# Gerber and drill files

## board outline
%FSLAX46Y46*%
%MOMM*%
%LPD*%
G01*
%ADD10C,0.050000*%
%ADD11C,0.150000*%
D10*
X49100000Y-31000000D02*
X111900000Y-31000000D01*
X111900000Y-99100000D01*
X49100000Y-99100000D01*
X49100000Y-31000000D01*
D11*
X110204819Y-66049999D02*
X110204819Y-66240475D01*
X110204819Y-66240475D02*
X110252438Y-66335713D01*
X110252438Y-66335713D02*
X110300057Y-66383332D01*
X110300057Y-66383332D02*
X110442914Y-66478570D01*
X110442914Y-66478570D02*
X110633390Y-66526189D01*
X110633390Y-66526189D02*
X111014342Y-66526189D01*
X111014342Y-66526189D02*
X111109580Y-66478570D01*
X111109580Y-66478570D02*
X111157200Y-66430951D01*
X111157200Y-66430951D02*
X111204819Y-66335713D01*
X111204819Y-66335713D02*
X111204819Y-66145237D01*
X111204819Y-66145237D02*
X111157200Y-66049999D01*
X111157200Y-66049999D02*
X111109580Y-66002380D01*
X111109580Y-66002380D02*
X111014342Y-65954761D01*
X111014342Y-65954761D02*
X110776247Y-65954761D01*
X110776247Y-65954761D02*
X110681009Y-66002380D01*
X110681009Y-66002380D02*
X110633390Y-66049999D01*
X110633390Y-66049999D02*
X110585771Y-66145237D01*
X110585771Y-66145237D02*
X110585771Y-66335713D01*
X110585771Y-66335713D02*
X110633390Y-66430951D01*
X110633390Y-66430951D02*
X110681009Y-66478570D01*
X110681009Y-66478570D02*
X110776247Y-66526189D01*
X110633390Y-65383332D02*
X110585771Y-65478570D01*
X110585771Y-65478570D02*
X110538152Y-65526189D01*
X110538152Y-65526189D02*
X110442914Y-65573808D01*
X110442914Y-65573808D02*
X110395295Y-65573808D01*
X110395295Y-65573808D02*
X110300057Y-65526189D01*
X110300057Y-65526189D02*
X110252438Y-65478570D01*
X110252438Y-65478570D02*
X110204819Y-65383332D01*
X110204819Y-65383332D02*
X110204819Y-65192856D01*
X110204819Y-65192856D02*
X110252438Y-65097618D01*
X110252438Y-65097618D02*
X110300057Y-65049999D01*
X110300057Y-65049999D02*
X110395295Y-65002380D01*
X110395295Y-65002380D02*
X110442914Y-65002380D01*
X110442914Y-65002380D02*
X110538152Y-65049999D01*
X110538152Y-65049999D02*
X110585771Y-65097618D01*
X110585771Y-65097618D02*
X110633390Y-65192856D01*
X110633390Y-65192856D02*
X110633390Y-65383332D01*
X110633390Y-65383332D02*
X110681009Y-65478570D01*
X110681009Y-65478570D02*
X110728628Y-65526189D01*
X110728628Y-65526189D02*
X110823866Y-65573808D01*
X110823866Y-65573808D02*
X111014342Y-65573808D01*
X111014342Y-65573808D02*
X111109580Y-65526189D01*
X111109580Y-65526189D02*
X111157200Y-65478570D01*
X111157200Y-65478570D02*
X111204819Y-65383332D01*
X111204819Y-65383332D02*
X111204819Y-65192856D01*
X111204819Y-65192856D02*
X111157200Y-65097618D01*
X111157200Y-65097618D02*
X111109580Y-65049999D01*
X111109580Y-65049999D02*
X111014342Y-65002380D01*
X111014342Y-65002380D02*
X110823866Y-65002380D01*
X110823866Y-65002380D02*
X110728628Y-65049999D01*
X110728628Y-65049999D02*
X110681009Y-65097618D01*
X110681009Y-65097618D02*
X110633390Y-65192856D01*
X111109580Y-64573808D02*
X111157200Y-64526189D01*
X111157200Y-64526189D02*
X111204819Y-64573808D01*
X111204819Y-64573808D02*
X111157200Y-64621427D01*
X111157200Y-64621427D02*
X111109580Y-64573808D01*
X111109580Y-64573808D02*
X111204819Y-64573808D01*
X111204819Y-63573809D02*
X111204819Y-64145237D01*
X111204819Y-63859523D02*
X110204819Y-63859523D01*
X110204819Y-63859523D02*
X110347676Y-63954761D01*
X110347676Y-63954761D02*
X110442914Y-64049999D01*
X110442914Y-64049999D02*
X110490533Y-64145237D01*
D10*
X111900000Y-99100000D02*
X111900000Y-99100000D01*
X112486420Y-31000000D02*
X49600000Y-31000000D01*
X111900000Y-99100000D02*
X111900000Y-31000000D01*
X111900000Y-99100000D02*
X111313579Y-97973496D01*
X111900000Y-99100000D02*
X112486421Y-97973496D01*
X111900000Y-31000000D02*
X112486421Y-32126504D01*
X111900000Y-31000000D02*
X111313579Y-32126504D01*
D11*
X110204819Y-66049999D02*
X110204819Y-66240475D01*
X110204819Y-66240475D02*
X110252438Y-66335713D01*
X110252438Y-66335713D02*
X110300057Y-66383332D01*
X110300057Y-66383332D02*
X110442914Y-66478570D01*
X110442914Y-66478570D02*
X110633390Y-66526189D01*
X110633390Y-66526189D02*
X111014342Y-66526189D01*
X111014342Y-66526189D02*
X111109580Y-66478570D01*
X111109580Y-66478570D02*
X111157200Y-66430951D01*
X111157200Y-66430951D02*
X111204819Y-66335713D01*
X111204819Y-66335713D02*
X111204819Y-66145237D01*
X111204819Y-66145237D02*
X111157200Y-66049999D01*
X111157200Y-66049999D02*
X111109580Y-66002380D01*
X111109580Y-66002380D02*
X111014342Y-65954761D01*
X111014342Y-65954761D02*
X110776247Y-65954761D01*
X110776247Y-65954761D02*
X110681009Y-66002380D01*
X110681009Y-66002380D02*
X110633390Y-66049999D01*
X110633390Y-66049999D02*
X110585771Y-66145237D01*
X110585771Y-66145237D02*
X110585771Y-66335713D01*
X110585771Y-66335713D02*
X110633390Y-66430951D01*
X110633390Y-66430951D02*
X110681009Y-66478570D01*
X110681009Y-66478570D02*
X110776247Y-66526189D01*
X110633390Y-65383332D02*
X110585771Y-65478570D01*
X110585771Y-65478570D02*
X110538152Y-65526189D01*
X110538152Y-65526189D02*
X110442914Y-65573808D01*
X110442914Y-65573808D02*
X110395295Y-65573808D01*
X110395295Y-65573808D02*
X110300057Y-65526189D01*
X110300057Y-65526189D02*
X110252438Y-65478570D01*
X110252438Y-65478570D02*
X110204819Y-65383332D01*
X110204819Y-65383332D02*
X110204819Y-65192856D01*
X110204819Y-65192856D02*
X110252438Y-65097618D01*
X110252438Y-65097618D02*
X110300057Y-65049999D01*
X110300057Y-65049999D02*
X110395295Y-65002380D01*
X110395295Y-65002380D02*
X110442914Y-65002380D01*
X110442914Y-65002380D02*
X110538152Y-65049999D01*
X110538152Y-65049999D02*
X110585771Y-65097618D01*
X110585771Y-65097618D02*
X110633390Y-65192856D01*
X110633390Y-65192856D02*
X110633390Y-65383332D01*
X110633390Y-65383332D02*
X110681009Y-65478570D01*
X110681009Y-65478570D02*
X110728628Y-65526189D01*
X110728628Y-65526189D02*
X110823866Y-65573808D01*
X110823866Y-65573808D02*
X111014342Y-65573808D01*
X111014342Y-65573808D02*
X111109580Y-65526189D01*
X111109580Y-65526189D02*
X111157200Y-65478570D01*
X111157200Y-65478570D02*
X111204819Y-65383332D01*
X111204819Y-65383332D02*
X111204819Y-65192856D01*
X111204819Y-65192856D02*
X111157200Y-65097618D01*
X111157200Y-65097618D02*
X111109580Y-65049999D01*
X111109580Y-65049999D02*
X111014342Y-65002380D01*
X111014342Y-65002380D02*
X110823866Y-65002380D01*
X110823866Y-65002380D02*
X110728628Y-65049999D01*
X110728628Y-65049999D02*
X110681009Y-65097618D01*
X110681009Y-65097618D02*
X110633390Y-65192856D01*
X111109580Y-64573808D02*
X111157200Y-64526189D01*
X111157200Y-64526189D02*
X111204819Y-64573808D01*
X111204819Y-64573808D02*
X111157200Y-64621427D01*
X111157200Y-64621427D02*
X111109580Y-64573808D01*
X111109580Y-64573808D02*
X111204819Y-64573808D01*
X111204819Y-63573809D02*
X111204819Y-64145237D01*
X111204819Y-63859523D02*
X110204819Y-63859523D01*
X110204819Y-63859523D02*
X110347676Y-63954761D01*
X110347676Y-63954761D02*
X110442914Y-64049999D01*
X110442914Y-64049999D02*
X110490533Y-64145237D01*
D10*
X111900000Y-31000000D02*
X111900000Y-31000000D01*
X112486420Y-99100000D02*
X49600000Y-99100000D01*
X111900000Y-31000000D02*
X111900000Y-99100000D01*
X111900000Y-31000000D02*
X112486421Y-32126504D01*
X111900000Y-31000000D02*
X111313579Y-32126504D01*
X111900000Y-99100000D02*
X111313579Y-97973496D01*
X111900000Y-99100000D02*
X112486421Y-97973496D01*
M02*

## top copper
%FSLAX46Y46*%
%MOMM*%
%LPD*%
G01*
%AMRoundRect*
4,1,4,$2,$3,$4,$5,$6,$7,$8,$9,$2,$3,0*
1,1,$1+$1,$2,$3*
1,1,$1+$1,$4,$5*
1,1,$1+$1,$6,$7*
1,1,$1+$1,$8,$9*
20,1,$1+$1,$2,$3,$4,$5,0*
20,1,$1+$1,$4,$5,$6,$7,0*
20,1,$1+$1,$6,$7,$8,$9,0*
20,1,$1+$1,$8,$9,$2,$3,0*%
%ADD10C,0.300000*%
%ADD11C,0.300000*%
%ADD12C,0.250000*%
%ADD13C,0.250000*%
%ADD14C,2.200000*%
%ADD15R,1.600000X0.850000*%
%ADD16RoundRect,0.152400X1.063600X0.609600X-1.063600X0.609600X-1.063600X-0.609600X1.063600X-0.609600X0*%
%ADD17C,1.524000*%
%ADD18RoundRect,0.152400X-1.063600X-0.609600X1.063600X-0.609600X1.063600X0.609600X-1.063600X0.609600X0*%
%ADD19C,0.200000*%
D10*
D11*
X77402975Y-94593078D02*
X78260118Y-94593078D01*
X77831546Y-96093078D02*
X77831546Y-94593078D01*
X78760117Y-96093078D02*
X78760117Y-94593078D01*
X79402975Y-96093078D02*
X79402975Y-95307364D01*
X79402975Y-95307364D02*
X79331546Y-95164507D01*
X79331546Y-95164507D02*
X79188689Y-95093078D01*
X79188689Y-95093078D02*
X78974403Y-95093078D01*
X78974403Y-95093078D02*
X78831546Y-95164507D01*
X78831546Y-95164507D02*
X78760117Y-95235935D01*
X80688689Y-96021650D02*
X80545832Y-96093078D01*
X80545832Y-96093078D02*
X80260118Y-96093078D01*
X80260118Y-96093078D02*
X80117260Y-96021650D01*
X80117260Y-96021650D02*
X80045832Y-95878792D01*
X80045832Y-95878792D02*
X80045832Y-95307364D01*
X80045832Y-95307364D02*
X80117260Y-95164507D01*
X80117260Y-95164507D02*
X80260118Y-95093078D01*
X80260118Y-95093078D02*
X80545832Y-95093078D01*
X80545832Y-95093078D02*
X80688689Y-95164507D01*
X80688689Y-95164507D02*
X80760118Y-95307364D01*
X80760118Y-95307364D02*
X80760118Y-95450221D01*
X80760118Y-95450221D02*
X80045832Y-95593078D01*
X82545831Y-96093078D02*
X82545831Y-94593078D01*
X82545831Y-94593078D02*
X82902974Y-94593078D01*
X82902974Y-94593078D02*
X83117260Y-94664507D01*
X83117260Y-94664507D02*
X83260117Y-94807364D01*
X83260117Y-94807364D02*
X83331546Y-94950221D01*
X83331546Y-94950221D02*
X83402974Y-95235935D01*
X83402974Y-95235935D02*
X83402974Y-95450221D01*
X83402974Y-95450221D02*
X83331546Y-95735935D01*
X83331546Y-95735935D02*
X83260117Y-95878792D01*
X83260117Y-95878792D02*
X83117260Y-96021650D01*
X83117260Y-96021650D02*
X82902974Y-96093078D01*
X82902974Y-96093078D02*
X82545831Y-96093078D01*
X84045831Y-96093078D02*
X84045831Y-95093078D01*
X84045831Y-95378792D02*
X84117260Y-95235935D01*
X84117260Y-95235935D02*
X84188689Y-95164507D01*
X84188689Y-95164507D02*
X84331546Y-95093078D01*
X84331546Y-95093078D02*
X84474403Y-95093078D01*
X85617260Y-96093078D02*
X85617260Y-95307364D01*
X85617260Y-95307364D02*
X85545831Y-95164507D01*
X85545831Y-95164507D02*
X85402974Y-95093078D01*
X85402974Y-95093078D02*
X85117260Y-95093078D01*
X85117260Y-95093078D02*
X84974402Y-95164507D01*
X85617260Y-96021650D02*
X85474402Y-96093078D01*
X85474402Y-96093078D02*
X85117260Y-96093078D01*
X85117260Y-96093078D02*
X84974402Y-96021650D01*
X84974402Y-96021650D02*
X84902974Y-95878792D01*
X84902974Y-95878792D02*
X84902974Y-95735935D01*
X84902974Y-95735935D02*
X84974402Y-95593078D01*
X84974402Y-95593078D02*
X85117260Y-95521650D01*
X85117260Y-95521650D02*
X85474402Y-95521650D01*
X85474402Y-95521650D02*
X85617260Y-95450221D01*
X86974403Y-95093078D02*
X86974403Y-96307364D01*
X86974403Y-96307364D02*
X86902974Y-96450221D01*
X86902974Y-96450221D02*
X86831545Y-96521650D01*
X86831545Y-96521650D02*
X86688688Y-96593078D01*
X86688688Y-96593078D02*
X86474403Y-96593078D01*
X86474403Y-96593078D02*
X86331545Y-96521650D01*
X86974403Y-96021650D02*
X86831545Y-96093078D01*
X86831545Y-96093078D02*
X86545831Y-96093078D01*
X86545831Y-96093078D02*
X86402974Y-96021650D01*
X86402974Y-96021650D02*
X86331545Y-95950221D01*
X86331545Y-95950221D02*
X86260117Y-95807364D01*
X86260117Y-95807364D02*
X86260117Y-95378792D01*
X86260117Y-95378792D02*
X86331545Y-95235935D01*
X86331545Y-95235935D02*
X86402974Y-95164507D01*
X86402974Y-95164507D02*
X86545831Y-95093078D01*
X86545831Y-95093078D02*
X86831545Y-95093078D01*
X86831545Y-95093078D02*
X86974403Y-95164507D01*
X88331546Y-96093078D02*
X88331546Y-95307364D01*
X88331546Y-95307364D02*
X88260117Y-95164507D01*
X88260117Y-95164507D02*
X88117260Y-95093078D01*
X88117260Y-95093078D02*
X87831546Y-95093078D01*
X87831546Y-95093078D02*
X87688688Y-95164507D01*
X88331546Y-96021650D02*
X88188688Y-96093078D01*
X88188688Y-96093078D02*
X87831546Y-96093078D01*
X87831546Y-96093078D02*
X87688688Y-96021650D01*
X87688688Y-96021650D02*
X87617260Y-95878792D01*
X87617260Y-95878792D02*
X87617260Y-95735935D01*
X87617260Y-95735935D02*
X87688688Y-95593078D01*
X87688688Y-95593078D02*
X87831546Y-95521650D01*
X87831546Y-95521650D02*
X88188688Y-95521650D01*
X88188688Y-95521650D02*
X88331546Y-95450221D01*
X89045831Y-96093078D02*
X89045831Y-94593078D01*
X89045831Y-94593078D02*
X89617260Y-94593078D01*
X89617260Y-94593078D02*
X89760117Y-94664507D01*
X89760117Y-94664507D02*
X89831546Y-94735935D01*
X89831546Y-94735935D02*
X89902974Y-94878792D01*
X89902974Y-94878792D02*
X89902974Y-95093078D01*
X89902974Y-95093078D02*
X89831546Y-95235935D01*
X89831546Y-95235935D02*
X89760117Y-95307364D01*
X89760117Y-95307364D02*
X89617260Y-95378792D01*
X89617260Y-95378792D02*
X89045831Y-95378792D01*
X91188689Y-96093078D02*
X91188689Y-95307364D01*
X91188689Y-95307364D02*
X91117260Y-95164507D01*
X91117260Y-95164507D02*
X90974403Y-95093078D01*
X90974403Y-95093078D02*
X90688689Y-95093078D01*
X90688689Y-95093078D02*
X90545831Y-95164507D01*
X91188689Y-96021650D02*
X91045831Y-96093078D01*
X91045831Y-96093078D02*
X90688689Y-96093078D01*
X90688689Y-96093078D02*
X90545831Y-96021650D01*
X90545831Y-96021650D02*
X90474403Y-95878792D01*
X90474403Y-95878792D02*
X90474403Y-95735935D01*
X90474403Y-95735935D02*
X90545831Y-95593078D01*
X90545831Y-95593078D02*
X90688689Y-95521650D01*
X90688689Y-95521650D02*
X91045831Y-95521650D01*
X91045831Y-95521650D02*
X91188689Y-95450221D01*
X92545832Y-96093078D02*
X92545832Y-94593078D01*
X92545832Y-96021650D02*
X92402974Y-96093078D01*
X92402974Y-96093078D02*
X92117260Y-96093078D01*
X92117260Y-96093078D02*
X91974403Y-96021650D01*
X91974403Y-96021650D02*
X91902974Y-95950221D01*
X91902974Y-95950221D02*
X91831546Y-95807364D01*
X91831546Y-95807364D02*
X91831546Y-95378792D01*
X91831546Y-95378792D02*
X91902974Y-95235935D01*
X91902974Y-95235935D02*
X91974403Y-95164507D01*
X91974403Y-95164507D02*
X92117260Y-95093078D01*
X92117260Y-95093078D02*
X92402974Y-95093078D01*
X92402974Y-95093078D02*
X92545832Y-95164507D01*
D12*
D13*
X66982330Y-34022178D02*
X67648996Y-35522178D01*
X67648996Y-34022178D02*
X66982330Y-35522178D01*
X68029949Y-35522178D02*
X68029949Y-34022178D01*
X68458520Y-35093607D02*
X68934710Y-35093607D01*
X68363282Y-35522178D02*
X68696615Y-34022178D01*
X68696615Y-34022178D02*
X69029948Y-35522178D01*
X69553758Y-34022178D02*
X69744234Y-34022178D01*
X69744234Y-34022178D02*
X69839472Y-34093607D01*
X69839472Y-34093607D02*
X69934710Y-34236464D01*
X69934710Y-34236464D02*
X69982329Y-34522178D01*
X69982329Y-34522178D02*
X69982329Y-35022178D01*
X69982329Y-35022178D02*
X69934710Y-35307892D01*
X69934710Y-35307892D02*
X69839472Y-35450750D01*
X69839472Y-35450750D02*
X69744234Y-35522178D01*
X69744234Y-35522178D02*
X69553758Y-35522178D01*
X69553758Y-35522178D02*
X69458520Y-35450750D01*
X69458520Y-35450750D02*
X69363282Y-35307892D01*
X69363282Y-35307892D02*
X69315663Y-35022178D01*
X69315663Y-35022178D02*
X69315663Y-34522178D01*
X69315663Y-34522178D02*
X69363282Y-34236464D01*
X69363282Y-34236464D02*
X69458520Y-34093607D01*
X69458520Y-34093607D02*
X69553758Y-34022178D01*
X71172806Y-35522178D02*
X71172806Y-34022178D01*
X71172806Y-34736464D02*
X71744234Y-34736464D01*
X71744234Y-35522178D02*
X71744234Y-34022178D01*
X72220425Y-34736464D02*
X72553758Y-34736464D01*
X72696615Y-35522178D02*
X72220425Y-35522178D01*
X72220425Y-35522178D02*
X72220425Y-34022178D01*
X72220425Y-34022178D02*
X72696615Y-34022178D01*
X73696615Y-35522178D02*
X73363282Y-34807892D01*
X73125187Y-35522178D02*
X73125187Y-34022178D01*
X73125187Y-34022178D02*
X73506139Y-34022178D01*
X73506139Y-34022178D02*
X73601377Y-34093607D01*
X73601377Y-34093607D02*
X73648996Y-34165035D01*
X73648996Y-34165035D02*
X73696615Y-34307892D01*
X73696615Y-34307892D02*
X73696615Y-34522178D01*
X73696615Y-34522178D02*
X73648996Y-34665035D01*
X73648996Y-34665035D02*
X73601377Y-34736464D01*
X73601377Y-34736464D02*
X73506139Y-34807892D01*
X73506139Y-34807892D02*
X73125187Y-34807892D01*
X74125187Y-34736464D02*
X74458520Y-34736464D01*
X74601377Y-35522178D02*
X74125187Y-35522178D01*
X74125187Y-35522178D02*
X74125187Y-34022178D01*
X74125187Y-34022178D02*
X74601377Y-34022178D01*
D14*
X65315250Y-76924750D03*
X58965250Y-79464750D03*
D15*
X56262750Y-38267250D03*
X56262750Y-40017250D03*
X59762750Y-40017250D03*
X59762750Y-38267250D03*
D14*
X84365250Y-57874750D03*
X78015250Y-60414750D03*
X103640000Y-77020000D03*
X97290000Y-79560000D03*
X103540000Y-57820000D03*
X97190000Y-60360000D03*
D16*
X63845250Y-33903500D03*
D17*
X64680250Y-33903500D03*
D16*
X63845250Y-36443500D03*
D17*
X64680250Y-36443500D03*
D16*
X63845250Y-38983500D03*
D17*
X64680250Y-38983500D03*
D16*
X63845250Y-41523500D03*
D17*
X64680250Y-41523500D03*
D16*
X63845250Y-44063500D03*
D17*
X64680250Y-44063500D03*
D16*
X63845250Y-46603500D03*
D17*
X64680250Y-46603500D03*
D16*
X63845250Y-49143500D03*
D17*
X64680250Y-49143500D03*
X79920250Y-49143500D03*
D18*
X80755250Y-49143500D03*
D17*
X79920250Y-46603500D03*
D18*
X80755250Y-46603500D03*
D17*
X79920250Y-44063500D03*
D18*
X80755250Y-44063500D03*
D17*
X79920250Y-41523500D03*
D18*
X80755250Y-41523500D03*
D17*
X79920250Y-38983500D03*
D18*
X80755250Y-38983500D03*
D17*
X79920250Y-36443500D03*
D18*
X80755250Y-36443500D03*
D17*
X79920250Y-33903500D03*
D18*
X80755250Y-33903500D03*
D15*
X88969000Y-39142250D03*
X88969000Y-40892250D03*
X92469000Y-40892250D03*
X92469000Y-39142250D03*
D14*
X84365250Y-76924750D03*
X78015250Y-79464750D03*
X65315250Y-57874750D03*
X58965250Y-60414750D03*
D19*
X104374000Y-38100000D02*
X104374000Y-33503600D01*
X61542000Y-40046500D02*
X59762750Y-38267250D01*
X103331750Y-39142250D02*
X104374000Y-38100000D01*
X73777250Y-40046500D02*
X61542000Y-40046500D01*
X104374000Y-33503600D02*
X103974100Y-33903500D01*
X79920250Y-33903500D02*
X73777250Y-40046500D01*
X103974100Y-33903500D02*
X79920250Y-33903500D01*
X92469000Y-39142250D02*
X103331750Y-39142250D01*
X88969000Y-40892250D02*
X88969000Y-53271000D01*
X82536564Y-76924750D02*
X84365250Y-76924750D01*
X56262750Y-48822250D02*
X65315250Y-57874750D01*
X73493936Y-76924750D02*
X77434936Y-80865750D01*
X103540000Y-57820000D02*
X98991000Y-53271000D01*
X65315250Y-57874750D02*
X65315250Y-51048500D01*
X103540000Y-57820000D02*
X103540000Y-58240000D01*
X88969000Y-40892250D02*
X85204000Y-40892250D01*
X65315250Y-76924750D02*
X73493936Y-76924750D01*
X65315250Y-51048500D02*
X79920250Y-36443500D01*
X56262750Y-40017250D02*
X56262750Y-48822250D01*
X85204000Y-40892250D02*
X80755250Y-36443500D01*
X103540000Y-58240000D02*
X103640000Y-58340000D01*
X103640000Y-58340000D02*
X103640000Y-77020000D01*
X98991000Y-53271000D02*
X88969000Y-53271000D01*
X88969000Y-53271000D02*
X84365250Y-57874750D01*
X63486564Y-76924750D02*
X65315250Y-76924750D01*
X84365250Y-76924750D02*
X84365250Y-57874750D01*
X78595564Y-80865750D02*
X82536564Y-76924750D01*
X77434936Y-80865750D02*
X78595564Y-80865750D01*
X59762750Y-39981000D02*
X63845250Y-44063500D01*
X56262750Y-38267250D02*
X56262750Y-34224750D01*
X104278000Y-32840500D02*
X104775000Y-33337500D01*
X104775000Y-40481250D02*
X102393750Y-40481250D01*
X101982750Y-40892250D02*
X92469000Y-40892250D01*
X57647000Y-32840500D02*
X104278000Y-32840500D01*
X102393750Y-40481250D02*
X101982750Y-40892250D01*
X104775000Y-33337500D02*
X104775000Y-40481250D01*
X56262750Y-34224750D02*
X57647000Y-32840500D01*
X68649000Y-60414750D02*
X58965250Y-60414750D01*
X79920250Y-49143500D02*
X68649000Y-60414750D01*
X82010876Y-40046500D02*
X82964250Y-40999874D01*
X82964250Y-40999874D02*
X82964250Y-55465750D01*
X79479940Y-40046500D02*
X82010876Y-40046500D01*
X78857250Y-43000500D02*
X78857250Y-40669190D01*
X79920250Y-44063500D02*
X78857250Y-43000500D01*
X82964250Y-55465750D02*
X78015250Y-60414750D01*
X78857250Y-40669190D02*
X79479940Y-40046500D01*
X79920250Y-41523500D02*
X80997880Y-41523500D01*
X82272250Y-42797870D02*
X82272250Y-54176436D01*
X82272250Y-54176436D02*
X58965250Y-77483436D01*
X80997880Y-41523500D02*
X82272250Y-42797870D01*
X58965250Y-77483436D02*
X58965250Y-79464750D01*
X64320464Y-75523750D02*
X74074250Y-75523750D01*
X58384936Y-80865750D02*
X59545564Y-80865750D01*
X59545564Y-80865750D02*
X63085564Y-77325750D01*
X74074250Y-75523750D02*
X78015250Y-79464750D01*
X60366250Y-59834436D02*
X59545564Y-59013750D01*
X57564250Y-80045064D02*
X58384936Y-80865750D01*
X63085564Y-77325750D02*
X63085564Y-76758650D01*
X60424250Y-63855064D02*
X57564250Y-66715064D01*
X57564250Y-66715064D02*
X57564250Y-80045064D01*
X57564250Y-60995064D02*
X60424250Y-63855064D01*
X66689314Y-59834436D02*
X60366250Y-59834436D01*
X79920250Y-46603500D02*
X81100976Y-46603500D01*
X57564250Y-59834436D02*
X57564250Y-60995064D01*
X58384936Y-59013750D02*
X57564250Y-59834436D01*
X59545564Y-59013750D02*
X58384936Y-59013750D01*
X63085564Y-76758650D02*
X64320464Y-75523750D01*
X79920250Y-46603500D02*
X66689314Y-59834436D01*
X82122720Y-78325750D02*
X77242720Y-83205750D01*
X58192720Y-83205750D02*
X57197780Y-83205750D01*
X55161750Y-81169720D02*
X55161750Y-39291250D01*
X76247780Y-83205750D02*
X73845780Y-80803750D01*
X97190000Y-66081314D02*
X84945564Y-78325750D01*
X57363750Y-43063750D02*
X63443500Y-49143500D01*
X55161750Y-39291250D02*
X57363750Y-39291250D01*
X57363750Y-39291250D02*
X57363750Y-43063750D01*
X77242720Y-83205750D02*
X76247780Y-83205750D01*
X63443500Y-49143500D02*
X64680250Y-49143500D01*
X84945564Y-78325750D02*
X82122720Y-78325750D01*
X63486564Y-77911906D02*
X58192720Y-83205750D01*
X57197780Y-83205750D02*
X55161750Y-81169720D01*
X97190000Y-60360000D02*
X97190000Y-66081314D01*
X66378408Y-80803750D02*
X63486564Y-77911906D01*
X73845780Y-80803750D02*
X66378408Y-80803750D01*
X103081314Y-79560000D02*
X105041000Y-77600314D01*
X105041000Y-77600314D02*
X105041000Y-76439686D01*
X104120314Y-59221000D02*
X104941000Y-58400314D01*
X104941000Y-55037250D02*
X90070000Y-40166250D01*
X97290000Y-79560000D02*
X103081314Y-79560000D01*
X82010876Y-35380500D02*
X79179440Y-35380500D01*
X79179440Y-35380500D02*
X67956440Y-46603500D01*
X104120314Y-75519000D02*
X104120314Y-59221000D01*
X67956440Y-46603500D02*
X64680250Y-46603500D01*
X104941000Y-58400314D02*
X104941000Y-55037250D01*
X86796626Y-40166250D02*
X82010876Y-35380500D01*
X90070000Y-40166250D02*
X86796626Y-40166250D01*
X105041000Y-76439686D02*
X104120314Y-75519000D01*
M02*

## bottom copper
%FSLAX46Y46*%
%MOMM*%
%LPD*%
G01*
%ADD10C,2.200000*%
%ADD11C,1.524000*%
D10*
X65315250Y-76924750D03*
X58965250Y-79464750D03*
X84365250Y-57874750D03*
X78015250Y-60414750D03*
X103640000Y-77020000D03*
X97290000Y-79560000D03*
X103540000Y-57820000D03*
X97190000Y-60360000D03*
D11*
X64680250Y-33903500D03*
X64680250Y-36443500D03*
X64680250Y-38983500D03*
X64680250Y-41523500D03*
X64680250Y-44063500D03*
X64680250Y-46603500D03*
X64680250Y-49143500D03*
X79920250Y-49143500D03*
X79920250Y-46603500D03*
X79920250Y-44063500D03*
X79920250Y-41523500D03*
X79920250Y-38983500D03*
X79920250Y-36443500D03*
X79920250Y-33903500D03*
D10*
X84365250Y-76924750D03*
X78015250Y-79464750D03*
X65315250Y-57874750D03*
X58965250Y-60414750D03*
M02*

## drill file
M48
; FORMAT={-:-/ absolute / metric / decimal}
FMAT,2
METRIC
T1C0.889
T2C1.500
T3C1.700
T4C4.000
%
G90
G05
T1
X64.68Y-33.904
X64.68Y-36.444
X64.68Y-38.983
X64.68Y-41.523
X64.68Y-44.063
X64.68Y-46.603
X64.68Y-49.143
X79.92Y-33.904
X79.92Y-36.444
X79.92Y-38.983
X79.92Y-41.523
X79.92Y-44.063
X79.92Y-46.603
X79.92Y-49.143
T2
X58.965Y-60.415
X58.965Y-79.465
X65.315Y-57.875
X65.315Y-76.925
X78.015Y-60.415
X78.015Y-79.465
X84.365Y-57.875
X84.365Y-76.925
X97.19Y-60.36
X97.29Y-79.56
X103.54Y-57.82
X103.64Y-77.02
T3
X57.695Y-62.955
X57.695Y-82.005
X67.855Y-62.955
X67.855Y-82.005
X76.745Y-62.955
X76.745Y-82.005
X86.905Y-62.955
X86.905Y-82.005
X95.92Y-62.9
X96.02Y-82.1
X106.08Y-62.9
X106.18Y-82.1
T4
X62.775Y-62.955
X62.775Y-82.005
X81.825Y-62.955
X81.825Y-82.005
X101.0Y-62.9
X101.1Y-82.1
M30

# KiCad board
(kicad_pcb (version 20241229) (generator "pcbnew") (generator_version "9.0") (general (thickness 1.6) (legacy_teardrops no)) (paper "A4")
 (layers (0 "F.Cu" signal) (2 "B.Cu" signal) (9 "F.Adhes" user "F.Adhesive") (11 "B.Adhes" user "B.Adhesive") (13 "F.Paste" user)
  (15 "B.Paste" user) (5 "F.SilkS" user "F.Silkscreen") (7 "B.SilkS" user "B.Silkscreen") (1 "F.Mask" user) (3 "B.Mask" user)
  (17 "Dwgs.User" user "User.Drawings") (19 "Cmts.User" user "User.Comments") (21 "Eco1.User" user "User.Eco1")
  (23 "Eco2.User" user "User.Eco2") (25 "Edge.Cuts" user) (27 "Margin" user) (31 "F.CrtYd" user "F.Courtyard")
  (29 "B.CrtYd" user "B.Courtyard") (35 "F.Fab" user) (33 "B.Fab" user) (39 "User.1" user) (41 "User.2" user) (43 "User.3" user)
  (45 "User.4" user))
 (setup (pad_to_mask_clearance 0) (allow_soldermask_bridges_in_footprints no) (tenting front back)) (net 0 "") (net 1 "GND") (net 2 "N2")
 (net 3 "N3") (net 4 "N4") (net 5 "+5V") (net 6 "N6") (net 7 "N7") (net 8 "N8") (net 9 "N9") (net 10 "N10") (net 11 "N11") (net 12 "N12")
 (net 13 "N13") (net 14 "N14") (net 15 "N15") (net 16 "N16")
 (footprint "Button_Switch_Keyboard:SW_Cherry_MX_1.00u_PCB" (layer "F.Cu") (at 65.31525 76.92475)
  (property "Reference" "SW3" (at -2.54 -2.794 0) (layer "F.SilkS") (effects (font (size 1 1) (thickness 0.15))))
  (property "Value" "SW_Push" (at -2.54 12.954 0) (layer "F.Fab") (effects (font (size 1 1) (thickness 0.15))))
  (pad "" np_thru_hole circle (at -7.62 5.08) (size 1.7 1.7) (drill 1.7) (layers "*.Cu" "*.Mask"))
  (pad "" np_thru_hole circle (at -2.54 5.08) (size 4 4) (drill 4) (layers "*.Cu" "*.Mask"))
  (pad "" np_thru_hole circle (at 2.54 5.08) (size 1.7 1.7) (drill 1.7) (layers "*.Cu" "*.Mask"))
  (pad "1" thru_hole circle (at 0 0) (size 2.2 2.2) (drill 1.5) (layers "*.Cu" "*.Mask") (remove_unused_layers no) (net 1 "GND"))
  (pad "2" thru_hole circle (at -6.35 2.54) (size 2.2 2.2) (drill 1.5) (layers "*.Cu" "*.Mask") (remove_unused_layers no) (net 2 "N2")))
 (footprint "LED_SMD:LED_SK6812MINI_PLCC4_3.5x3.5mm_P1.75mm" (layer "F.Cu") (at 58.01275 39.14225)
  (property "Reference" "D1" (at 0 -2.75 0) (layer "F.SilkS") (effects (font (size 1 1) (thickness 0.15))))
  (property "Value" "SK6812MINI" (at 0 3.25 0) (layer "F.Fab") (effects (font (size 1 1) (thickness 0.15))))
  (pad "1" smd rect (at -1.75 -0.875) (size 1.6 0.85) (layers "F.Cu" "F.Mask" "F.Paste") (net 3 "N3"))
  (pad "2" smd rect (at -1.75 0.875) (size 1.6 0.85) (layers "F.Cu" "F.Mask" "F.Paste") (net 1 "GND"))
  (pad "3" smd rect (at 1.75 0.875) (size 1.6 0.85) (layers "F.Cu" "F.Mask" "F.Paste") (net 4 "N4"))
  (pad "4" smd rect (at 1.75 -0.875) (size 1.6 0.85) (layers "F.Cu" "F.Mask" "F.Paste") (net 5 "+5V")))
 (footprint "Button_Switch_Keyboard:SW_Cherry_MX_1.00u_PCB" (layer "F.Cu") (at 84.36525 57.87475)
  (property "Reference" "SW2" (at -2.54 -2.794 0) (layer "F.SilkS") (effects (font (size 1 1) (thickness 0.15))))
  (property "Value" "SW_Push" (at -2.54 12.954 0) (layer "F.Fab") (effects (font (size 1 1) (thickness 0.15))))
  (pad "" np_thru_hole circle (at -7.62 5.08) (size 1.7 1.7) (drill 1.7) (layers "*.Cu" "*.Mask"))
  (pad "" np_thru_hole circle (at -2.54 5.08) (size 4 4) (drill 4) (layers "*.Cu" "*.Mask"))
  (pad "" np_thru_hole circle (at 2.54 5.08) (size 1.7 1.7) (drill 1.7) (layers "*.Cu" "*.Mask"))
  (pad "1" thru_hole circle (at 0 0) (size 2.2 2.2) (drill 1.5) (layers "*.Cu" "*.Mask") (remove_unused_layers no) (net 1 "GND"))
  (pad "2" thru_hole circle (at -6.35 2.54) (size 2.2 2.2) (drill 1.5) (layers "*.Cu" "*.Mask") (remove_unused_layers no) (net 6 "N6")))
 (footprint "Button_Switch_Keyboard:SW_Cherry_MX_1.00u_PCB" (layer "F.Cu") (at 103.64 77.02)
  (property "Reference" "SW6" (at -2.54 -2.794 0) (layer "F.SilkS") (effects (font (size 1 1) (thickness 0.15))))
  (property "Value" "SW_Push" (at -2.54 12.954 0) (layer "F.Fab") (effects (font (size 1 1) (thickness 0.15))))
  (pad "" np_thru_hole circle (at -7.62 5.08) (size 1.7 1.7) (drill 1.7) (layers "*.Cu" "*.Mask"))
  (pad "" np_thru_hole circle (at -2.54 5.08) (size 4 4) (drill 4) (layers "*.Cu" "*.Mask"))
  (pad "" np_thru_hole circle (at 2.54 5.08) (size 1.7 1.7) (drill 1.7) (layers "*.Cu" "*.Mask"))
  (pad "1" thru_hole circle (at 0 0) (size 2.2 2.2) (drill 1.5) (layers "*.Cu" "*.Mask") (remove_unused_layers no) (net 1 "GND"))
  (pad "2" thru_hole circle (at -6.35 2.54) (size 2.2 2.2) (drill 1.5) (layers "*.Cu" "*.Mask") (remove_unused_layers no) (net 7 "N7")))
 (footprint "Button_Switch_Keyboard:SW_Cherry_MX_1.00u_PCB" (layer "F.Cu") (at 103.54 57.82)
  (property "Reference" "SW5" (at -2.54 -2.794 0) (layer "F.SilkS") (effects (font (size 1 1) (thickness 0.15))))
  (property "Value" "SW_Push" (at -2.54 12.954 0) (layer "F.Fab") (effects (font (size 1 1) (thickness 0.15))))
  (pad "" np_thru_hole circle (at -7.62 5.08) (size 1.7 1.7) (drill 1.7) (layers "*.Cu" "*.Mask"))
  (pad "" np_thru_hole circle (at -2.54 5.08) (size 4 4) (drill 4) (layers "*.Cu" "*.Mask"))
  (pad "" np_thru_hole circle (at 2.54 5.08) (size 1.7 1.7) (drill 1.7) (layers "*.Cu" "*.Mask"))
  (pad "1" thru_hole circle (at 0 0) (size 2.2 2.2) (drill 1.5) (layers "*.Cu" "*.Mask") (remove_unused_layers no) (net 1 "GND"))
  (pad "2" thru_hole circle (at -6.35 2.54) (size 2.2 2.2) (drill 1.5) (layers "*.Cu" "*.Mask") (remove_unused_layers no) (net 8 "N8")))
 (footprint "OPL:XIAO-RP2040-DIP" (layer "F.Cu") (at 72.30025 41.5235)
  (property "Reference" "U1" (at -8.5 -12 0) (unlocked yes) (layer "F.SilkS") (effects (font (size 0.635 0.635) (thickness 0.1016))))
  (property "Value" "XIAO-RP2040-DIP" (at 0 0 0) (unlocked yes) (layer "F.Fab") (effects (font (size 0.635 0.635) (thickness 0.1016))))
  (pad "1" smd roundrect (at -8.455 -7.62 180) (size 2.432 1.524) (layers "F.Cu" "F.Mask") (roundrect_rratio 0.1) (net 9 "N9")
   (thermal_bridge_angle 45))
  (pad "1" thru_hole circle (at -7.62 -7.62 180) (size 1.524 1.524) (drill 0.889) (layers "*.Cu" "*.Mask") (remove_unused_layers no)
   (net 9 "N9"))
  (pad "2" smd roundrect (at -8.455 -5.08 180) (size 2.432 1.524) (layers "F.Cu" "F.Mask") (roundrect_rratio 0.1) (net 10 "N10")
   (thermal_bridge_angle 45))
  (pad "2" thru_hole circle (at -7.62 -5.08 180) (size 1.524 1.524) (drill 0.889) (layers "*.Cu" "*.Mask") (remove_unused_layers no)
   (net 10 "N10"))
  (pad "3" smd roundrect (at -8.455 -2.54 180) (size 2.432 1.524) (layers "F.Cu" "F.Mask") (roundrect_rratio 0.1) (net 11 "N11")
   (thermal_bridge_angle 45))
  (pad "3" thru_hole circle (at -7.62 -2.54 180) (size 1.524 1.524) (drill 0.889) (layers "*.Cu" "*.Mask") (remove_unused_layers no)
   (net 11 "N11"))
  (pad "4" smd roundrect (at -8.455 0 180) (size 2.432 1.524) (layers "F.Cu" "F.Mask") (roundrect_rratio 0.1) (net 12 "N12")
   (thermal_bridge_angle 45))
  (pad "4" thru_hole circle (at -7.62 0 180) (size 1.524 1.524) (drill 0.889) (layers "*.Cu" "*.Mask") (remove_unused_layers no)
   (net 12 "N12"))
  (pad "5" smd roundrect (at -8.455 2.54 180) (size 2.432 1.524) (layers "F.Cu" "F.Mask") (roundrect_rratio 0.1) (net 4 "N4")
   (thermal_bridge_angle 45))
  (pad "5" thru_hole circle (at -7.62 2.54 180) (size 1.524 1.524) (drill 0.889) (layers "*.Cu" "*.Mask") (remove_unused_layers no)
   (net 4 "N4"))
  (pad "6" smd roundrect (at -8.455 5.08 180) (size 2.432 1.524) (layers "F.Cu" "F.Mask") (roundrect_rratio 0.1) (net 7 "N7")
   (thermal_bridge_angle 45))
  (pad "6" thru_hole circle (at -7.62 5.08 180) (size 1.524 1.524) (drill 0.889) (layers "*.Cu" "*.Mask") (remove_unused_layers no)
   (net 7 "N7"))
  (pad "7" smd roundrect (at -8.455 7.62 180) (size 2.432 1.524) (layers "F.Cu" "F.Mask") (roundrect_rratio 0.1) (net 8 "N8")
   (thermal_bridge_angle 45))
  (pad "7" thru_hole circle (at -7.62 7.62 180) (size 1.524 1.524) (drill 0.889) (layers "*.Cu" "*.Mask") (remove_unused_layers no)
   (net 8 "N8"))
  (pad "8" thru_hole circle (at 7.62 7.62) (size 1.524 1.524) (drill 0.889) (layers "*.Cu" "*.Mask") (remove_unused_layers no)
   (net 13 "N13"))
  (pad "8" smd roundrect (at 8.455 7.62) (size 2.432 1.524) (layers "F.Cu" "F.Mask") (roundrect_rratio 0.1) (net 13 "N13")
   (thermal_bridge_angle 45))
  (pad "9" thru_hole circle (at 7.62 5.08) (size 1.524 1.524) (drill 0.889) (layers "*.Cu" "*.Mask") (remove_unused_layers no)
   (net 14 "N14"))
  (pad "9" smd roundrect (at 8.455 5.08) (size 2.432 1.524) (layers "F.Cu" "F.Mask") (roundrect_rratio 0.1) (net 14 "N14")
   (thermal_bridge_angle 45))
  (pad "10" thru_hole circle (at 7.62 2.54) (size 1.524 1.524) (drill 0.889) (layers "*.Cu" "*.Mask") (remove_unused_layers no) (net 6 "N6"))
  (pad "10" smd roundrect (at 8.455 2.54) (size 2.432 1.524) (layers "F.Cu" "F.Mask") (roundrect_rratio 0.1) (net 6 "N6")
   (thermal_bridge_angle 45))
  (pad "11" thru_hole circle (at 7.62 0) (size 1.524 1.524) (drill 0.889) (layers "*.Cu" "*.Mask") (remove_unused_layers no) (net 2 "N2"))
  (pad "11" smd roundrect (at 8.455 0) (size 2.432 1.524) (layers "F.Cu" "F.Mask") (roundrect_rratio 0.1) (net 2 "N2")
   (thermal_bridge_angle 45))
  (pad "12" thru_hole circle (at 7.62 -2.54) (size 1.524 1.524) (drill 0.889) (layers "*.Cu" "*.Mask") (remove_unused_layers no)
   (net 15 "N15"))
  (pad "12" smd roundrect (at 8.455 -2.54) (size 2.432 1.524) (layers "F.Cu" "F.Mask") (roundrect_rratio 0.1) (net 15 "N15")
   (thermal_bridge_angle 45))
  (pad "13" thru_hole circle (at 7.62 -5.08) (size 1.524 1.524) (drill 0.889) (layers "*.Cu" "*.Mask") (remove_unused_layers no)
   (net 1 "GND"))
  (pad "13" smd roundrect (at 8.455 -5.08) (size 2.432 1.524) (layers "F.Cu" "F.Mask") (roundrect_rratio 0.1) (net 1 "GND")
   (thermal_bridge_angle 45))
  (pad "14" thru_hole circle (at 7.62 -7.62) (size 1.524 1.524) (drill 0.889) (layers "*.Cu" "*.Mask") (remove_unused_layers no)
   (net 5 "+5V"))
  (pad "14" smd roundrect (at 8.455 -7.62) (size 2.432 1.524) (layers "F.Cu" "F.Mask") (roundrect_rratio 0.1) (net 5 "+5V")
   (thermal_bridge_angle 45)))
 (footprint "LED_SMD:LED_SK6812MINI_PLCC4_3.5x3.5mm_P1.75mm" (layer "F.Cu") (at 90.719 40.01725)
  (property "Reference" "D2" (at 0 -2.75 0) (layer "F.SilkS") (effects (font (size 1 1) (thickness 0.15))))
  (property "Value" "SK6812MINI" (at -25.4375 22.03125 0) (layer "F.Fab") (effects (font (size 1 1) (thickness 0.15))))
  (pad "1" smd rect (at -1.75 -0.875) (size 1.6 0.85) (layers "F.Cu" "F.Mask" "F.Paste") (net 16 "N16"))
  (pad "2" smd rect (at -1.75 0.875) (size 1.6 0.85) (layers "F.Cu" "F.Mask" "F.Paste") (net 1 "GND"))
  (pad "3" smd rect (at 1.75 0.875) (size 1.6 0.85) (layers "F.Cu" "F.Mask" "F.Paste") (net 3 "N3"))
  (pad "4" smd rect (at 1.75 -0.875) (size 1.6 0.85) (layers "F.Cu" "F.Mask" "F.Paste") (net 5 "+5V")))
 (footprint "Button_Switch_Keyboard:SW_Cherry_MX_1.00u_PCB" (layer "F.Cu") (at 84.36525 76.92475)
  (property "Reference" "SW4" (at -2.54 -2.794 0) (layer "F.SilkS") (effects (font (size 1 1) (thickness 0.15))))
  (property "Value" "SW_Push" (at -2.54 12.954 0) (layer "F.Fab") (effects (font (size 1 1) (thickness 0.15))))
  (pad "" np_thru_hole circle (at -7.62 5.08) (size 1.7 1.7) (drill 1.7) (layers "*.Cu" "*.Mask"))
  (pad "" np_thru_hole circle (at -2.54 5.08) (size 4 4) (drill 4) (layers "*.Cu" "*.Mask"))
  (pad "" np_thru_hole circle (at 2.54 5.08) (size 1.7 1.7) (drill 1.7) (layers "*.Cu" "*.Mask"))
  (pad "1" thru_hole circle (at 0 0) (size 2.2 2.2) (drill 1.5) (layers "*.Cu" "*.Mask") (remove_unused_layers no) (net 1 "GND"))
  (pad "2" thru_hole circle (at -6.35 2.54) (size 2.2 2.2) (drill 1.5) (layers "*.Cu" "*.Mask") (remove_unused_layers no) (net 14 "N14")))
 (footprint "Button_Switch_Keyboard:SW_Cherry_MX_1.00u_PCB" (layer "F.Cu") (at 65.31525 57.87475)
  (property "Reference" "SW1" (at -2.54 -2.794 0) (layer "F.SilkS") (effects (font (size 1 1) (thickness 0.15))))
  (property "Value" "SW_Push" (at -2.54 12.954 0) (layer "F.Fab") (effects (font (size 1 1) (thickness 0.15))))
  (pad "" np_thru_hole circle (at -7.62 5.08) (size 1.7 1.7) (drill 1.7) (layers "*.Cu" "*.Mask"))
  (pad "" np_thru_hole circle (at -2.54 5.08) (size 4 4) (drill 4) (layers "*.Cu" "*.Mask"))
  (pad "" np_thru_hole circle (at 2.54 5.08) (size 1.7 1.7) (drill 1.7) (layers "*.Cu" "*.Mask"))
  (pad "1" thru_hole circle (at 0 0) (size 2.2 2.2) (drill 1.5) (layers "*.Cu" "*.Mask") (remove_unused_layers no) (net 1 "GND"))
  (pad "2" thru_hole circle (at -6.35 2.54) (size 2.2 2.2) (drill 1.5) (layers "*.Cu" "*.Mask") (remove_unused_layers no) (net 13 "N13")))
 (gr_rect (start 49.1 31) (end 111.9 99.1) (stroke (width 0.05) (type default)) (fill no) (layer "Edge.Cuts"))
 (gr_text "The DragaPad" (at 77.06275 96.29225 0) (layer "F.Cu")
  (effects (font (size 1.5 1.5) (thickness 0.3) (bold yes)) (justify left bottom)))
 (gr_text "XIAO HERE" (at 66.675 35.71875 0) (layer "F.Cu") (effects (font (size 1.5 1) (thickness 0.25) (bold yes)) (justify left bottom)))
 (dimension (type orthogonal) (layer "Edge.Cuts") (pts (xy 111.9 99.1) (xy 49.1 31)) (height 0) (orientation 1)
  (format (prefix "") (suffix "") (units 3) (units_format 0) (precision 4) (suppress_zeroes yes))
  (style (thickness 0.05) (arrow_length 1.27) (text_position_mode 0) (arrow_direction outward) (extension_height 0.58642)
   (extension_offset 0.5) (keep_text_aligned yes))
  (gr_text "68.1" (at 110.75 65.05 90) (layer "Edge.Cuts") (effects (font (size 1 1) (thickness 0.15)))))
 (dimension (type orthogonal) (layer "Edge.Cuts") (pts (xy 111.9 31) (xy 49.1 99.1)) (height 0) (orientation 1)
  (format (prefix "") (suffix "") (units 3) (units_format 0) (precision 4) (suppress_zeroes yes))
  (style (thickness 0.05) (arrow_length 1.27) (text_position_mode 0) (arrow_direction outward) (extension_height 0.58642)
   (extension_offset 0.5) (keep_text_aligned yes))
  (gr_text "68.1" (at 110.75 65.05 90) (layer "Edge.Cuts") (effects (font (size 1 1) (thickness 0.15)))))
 (segment (start 104.374 38.1) (end 104.374 33.5036) (width 0.2) (layer "F.Cu") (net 5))
 (segment (start 61.542 40.0465) (end 59.76275 38.26725) (width 0.2) (layer "F.Cu") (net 5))
 (segment (start 103.33175 39.14225) (end 104.374 38.1) (width 0.2) (layer "F.Cu") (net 5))
 (segment (start 73.77725 40.0465) (end 61.542 40.0465) (width 0.2) (layer "F.Cu") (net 5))
 (segment (start 104.374 33.5036) (end 103.9741 33.9035) (width 0.2) (layer "F.Cu") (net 5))
 (segment (start 79.92025 33.9035) (end 73.77725 40.0465) (width 0.2) (layer "F.Cu") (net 5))
 (segment (start 103.9741 33.9035) (end 79.92025 33.9035) (width 0.2) (layer "F.Cu") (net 5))
 (segment (start 92.469 39.14225) (end 103.33175 39.14225) (width 0.2) (layer "F.Cu") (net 5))
 (segment (start 88.969 40.89225) (end 88.969 53.271) (width 0.2) (layer "F.Cu") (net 1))
 (segment (start 82.536564 76.92475) (end 84.36525 76.92475) (width 0.2) (layer "F.Cu") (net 1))
 (segment (start 56.26275 48.82225) (end 65.31525 57.87475) (width 0.2) (layer "F.Cu") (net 1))
 (segment (start 73.493936 76.92475) (end 77.434936 80.86575) (width 0.2) (layer "F.Cu") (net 1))
 (segment (start 103.54 57.82) (end 98.991 53.271) (width 0.2) (layer "F.Cu") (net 1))
 (segment (start 65.31525 57.87475) (end 65.31525 51.0485) (width 0.2) (layer "F.Cu") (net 1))
 (segment (start 103.54 57.82) (end 103.54 58.24) (width 0.2) (layer "F.Cu") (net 1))
 (segment (start 88.969 40.89225) (end 85.204 40.89225) (width 0.2) (layer "F.Cu") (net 1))
 (segment (start 65.31525 76.92475) (end 73.493936 76.92475) (width 0.2) (layer "F.Cu") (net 1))
 (segment (start 65.31525 51.0485) (end 79.92025 36.4435) (width 0.2) (layer "F.Cu") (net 1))
 (segment (start 56.26275 40.01725) (end 56.26275 48.82225) (width 0.2) (layer "F.Cu") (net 1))
 (segment (start 85.204 40.89225) (end 80.75525 36.4435) (width 0.2) (layer "F.Cu") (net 1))
 (segment (start 103.54 58.24) (end 103.64 58.34) (width 0.2) (layer "F.Cu") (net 1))
 (segment (start 103.64 58.34) (end 103.64 77.02) (width 0.2) (layer "F.Cu") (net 1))
 (segment (start 98.991 53.271) (end 88.969 53.271) (width 0.2) (layer "F.Cu") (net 1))
 (segment (start 88.969 53.271) (end 84.36525 57.87475) (width 0.2) (layer "F.Cu") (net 1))
 (segment (start 63.486564 76.92475) (end 65.31525 76.92475) (width 0.2) (layer "F.Cu") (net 1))
 (segment (start 84.36525 76.92475) (end 84.36525 57.87475) (width 0.2) (layer "F.Cu") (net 1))
 (segment (start 78.595564 80.86575) (end 82.536564 76.92475) (width 0.2) (layer "F.Cu") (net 1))
 (segment (start 77.434936 80.86575) (end 78.595564 80.86575) (width 0.2) (layer "F.Cu") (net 1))
 (segment (start 59.76275 39.981) (end 63.84525 44.0635) (width 0.2) (layer "F.Cu") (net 4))
 (segment (start 56.26275 38.26725) (end 56.26275 34.22475) (width 0.2) (layer "F.Cu") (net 3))
 (segment (start 104.278 32.8405) (end 104.775 33.3375) (width 0.2) (layer "F.Cu") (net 3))
 (segment (start 104.775 40.48125) (end 102.39375 40.48125) (width 0.2) (layer "F.Cu") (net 3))
 (segment (start 101.98275 40.89225) (end 92.469 40.89225) (width 0.2) (layer "F.Cu") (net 3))
 (segment (start 57.647 32.8405) (end 104.278 32.8405) (width 0.2) (layer "F.Cu") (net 3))
 (segment (start 102.39375 40.48125) (end 101.98275 40.89225) (width 0.2) (layer "F.Cu") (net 3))
 (segment (start 104.775 33.3375) (end 104.775 40.48125) (width 0.2) (layer "F.Cu") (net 3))
 (segment (start 56.26275 34.22475) (end 57.647 32.8405) (width 0.2) (layer "F.Cu") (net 3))
 (segment (start 68.649 60.41475) (end 58.96525 60.41475) (width 0.2) (layer "F.Cu") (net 13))
 (segment (start 79.92025 49.1435) (end 68.649 60.41475) (width 0.2) (layer "F.Cu") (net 13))
 (segment (start 82.010876 40.0465) (end 82.96425 40.999874) (width 0.2) (layer "F.Cu") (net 6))
 (segment (start 82.96425 40.999874) (end 82.96425 55.46575) (width 0.2) (layer "F.Cu") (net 6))
 (segment (start 79.47994 40.0465) (end 82.010876 40.0465) (width 0.2) (layer "F.Cu") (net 6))
 (segment (start 78.85725 43.0005) (end 78.85725 40.66919) (width 0.2) (layer "F.Cu") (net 6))
 (segment (start 79.92025 44.0635) (end 78.85725 43.0005) (width 0.2) (layer "F.Cu") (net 6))
 (segment (start 82.96425 55.46575) (end 78.01525 60.41475) (width 0.2) (layer "F.Cu") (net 6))
 (segment (start 78.85725 40.66919) (end 79.47994 40.0465) (width 0.2) (layer "F.Cu") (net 6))
 (segment (start 79.92025 41.5235) (end 80.99788 41.5235) (width 0.2) (layer "F.Cu") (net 2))
 (segment (start 82.27225 42.79787) (end 82.27225 54.176436) (width 0.2) (layer "F.Cu") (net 2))
 (segment (start 82.27225 54.176436) (end 58.96525 77.483436) (width 0.2) (layer "F.Cu") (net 2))
 (segment (start 80.99788 41.5235) (end 82.27225 42.79787) (width 0.2) (layer "F.Cu") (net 2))
 (segment (start 58.96525 77.483436) (end 58.96525 79.46475) (width 0.2) (layer "F.Cu") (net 2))
 (segment (start 64.320464 75.52375) (end 74.07425 75.52375) (width 0.2) (layer "F.Cu") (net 14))
 (segment (start 58.384936 80.86575) (end 59.545564 80.86575) (width 0.2) (layer "F.Cu") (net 14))
 (segment (start 59.545564 80.86575) (end 63.085564 77.32575) (width 0.2) (layer "F.Cu") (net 14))
 (segment (start 74.07425 75.52375) (end 78.01525 79.46475) (width 0.2) (layer "F.Cu") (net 14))
 (segment (start 60.36625 59.834436) (end 59.545564 59.01375) (width 0.2) (layer "F.Cu") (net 14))
 (segment (start 57.56425 80.045064) (end 58.384936 80.86575) (width 0.2) (layer "F.Cu") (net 14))
 (segment (start 63.085564 77.32575) (end 63.085564 76.75865) (width 0.2) (layer "F.Cu") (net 14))
 (segment (start 60.42425 63.855064) (end 57.56425 66.715064) (width 0.2) (layer "F.Cu") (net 14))
 (segment (start 57.56425 66.715064) (end 57.56425 80.045064) (width 0.2) (layer "F.Cu") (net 14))
 (segment (start 57.56425 60.995064) (end 60.42425 63.855064) (width 0.2) (layer "F.Cu") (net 14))
 (segment (start 66.689314 59.834436) (end 60.36625 59.834436) (width 0.2) (layer "F.Cu") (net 14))
 (segment (start 79.92025 46.6035) (end 81.100976 46.6035) (width 0.2) (layer "F.Cu") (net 14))
 (segment (start 57.56425 59.834436) (end 57.56425 60.995064) (width 0.2) (layer "F.Cu") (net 14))
 (segment (start 58.384936 59.01375) (end 57.56425 59.834436) (width 0.2) (layer "F.Cu") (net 14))
 (segment (start 59.545564 59.01375) (end 58.384936 59.01375) (width 0.2) (layer "F.Cu") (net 14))
 (segment (start 63.085564 76.75865) (end 64.320464 75.52375) (width 0.2) (layer "F.Cu") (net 14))
 (segment (start 79.92025 46.6035) (end 66.689314 59.834436) (width 0.2) (layer "F.Cu") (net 14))
 (segment (start 82.12272 78.32575) (end 77.24272 83.20575) (width 0.2) (layer "F.Cu") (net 8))
 (segment (start 58.19272 83.20575) (end 57.19778 83.20575) (width 0.2) (layer "F.Cu") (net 8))
 (segment (start 55.16175 81.16972) (end 55.16175 39.29125) (width 0.2) (layer "F.Cu") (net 8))
 (segment (start 76.24778 83.20575) (end 73.84578 80.80375) (width 0.2) (layer "F.Cu") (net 8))
 (segment (start 97.19 66.081314) (end 84.945564 78.32575) (width 0.2) (layer "F.Cu") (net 8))
 (segment (start 57.36375 43.06375) (end 63.4435 49.1435) (width 0.2) (layer "F.Cu") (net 8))
 (segment (start 55.16175 39.29125) (end 57.36375 39.29125) (width 0.2) (layer "F.Cu") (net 8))
 (segment (start 57.36375 39.29125) (end 57.36375 43.06375) (width 0.2) (layer "F.Cu") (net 8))
 (segment (start 77.24272 83.20575) (end 76.24778 83.20575) (width 0.2) (layer "F.Cu") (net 8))
 (segment (start 63.4435 49.1435) (end 64.68025 49.1435) (width 0.2) (layer "F.Cu") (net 8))
 (segment (start 84.945564 78.32575) (end 82.12272 78.32575) (width 0.2) (layer "F.Cu") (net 8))
 (segment (start 63.486564 77.911906) (end 58.19272 83.20575) (width 0.2) (layer "F.Cu") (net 8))
 (segment (start 57.19778 83.20575) (end 55.16175 81.16972) (width 0.2) (layer "F.Cu") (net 8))
 (segment (start 97.19 60.36) (end 97.19 66.081314) (width 0.2) (layer "F.Cu") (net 8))
 (segment (start 66.378408 80.80375) (end 63.486564 77.911906) (width 0.2) (layer "F.Cu") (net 8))
 (segment (start 73.84578 80.80375) (end 66.378408 80.80375) (width 0.2) (layer "F.Cu") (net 8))
 (segment (start 103.081314 79.56) (end 105.041 77.600314) (width 0.2) (layer "F.Cu") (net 7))
 (segment (start 105.041 77.600314) (end 105.041 76.439686) (width 0.2) (layer "F.Cu") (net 7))
 (segment (start 104.120314 59.221) (end 104.941 58.400314) (width 0.2) (layer "F.Cu") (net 7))
 (segment (start 104.941 55.03725) (end 90.07 40.16625) (width 0.2) (layer "F.Cu") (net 7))
 (segment (start 97.29 79.56) (end 103.081314 79.56) (width 0.2) (layer "F.Cu") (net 7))
 (segment (start 82.010876 35.3805) (end 79.17944 35.3805) (width 0.2) (layer "F.Cu") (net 7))
 (segment (start 79.17944 35.3805) (end 67.95644 46.6035) (width 0.2) (layer "F.Cu") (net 7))
 (segment (start 104.120314 75.519) (end 104.120314 59.221) (width 0.2) (layer "F.Cu") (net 7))
 (segment (start 67.95644 46.6035) (end 64.68025 46.6035) (width 0.2) (layer "F.Cu") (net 7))
 (segment (start 104.941 58.400314) (end 104.941 55.03725) (width 0.2) (layer "F.Cu") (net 7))
 (segment (start 86.796626 40.16625) (end 82.010876 35.3805) (width 0.2) (layer "F.Cu") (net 7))
 (segment (start 90.07 40.16625) (end 86.796626 40.16625) (width 0.2) (layer "F.Cu") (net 7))
 (segment (start 105.041 76.439686) (end 104.120314 75.519) (width 0.2) (layer "F.Cu") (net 7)))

